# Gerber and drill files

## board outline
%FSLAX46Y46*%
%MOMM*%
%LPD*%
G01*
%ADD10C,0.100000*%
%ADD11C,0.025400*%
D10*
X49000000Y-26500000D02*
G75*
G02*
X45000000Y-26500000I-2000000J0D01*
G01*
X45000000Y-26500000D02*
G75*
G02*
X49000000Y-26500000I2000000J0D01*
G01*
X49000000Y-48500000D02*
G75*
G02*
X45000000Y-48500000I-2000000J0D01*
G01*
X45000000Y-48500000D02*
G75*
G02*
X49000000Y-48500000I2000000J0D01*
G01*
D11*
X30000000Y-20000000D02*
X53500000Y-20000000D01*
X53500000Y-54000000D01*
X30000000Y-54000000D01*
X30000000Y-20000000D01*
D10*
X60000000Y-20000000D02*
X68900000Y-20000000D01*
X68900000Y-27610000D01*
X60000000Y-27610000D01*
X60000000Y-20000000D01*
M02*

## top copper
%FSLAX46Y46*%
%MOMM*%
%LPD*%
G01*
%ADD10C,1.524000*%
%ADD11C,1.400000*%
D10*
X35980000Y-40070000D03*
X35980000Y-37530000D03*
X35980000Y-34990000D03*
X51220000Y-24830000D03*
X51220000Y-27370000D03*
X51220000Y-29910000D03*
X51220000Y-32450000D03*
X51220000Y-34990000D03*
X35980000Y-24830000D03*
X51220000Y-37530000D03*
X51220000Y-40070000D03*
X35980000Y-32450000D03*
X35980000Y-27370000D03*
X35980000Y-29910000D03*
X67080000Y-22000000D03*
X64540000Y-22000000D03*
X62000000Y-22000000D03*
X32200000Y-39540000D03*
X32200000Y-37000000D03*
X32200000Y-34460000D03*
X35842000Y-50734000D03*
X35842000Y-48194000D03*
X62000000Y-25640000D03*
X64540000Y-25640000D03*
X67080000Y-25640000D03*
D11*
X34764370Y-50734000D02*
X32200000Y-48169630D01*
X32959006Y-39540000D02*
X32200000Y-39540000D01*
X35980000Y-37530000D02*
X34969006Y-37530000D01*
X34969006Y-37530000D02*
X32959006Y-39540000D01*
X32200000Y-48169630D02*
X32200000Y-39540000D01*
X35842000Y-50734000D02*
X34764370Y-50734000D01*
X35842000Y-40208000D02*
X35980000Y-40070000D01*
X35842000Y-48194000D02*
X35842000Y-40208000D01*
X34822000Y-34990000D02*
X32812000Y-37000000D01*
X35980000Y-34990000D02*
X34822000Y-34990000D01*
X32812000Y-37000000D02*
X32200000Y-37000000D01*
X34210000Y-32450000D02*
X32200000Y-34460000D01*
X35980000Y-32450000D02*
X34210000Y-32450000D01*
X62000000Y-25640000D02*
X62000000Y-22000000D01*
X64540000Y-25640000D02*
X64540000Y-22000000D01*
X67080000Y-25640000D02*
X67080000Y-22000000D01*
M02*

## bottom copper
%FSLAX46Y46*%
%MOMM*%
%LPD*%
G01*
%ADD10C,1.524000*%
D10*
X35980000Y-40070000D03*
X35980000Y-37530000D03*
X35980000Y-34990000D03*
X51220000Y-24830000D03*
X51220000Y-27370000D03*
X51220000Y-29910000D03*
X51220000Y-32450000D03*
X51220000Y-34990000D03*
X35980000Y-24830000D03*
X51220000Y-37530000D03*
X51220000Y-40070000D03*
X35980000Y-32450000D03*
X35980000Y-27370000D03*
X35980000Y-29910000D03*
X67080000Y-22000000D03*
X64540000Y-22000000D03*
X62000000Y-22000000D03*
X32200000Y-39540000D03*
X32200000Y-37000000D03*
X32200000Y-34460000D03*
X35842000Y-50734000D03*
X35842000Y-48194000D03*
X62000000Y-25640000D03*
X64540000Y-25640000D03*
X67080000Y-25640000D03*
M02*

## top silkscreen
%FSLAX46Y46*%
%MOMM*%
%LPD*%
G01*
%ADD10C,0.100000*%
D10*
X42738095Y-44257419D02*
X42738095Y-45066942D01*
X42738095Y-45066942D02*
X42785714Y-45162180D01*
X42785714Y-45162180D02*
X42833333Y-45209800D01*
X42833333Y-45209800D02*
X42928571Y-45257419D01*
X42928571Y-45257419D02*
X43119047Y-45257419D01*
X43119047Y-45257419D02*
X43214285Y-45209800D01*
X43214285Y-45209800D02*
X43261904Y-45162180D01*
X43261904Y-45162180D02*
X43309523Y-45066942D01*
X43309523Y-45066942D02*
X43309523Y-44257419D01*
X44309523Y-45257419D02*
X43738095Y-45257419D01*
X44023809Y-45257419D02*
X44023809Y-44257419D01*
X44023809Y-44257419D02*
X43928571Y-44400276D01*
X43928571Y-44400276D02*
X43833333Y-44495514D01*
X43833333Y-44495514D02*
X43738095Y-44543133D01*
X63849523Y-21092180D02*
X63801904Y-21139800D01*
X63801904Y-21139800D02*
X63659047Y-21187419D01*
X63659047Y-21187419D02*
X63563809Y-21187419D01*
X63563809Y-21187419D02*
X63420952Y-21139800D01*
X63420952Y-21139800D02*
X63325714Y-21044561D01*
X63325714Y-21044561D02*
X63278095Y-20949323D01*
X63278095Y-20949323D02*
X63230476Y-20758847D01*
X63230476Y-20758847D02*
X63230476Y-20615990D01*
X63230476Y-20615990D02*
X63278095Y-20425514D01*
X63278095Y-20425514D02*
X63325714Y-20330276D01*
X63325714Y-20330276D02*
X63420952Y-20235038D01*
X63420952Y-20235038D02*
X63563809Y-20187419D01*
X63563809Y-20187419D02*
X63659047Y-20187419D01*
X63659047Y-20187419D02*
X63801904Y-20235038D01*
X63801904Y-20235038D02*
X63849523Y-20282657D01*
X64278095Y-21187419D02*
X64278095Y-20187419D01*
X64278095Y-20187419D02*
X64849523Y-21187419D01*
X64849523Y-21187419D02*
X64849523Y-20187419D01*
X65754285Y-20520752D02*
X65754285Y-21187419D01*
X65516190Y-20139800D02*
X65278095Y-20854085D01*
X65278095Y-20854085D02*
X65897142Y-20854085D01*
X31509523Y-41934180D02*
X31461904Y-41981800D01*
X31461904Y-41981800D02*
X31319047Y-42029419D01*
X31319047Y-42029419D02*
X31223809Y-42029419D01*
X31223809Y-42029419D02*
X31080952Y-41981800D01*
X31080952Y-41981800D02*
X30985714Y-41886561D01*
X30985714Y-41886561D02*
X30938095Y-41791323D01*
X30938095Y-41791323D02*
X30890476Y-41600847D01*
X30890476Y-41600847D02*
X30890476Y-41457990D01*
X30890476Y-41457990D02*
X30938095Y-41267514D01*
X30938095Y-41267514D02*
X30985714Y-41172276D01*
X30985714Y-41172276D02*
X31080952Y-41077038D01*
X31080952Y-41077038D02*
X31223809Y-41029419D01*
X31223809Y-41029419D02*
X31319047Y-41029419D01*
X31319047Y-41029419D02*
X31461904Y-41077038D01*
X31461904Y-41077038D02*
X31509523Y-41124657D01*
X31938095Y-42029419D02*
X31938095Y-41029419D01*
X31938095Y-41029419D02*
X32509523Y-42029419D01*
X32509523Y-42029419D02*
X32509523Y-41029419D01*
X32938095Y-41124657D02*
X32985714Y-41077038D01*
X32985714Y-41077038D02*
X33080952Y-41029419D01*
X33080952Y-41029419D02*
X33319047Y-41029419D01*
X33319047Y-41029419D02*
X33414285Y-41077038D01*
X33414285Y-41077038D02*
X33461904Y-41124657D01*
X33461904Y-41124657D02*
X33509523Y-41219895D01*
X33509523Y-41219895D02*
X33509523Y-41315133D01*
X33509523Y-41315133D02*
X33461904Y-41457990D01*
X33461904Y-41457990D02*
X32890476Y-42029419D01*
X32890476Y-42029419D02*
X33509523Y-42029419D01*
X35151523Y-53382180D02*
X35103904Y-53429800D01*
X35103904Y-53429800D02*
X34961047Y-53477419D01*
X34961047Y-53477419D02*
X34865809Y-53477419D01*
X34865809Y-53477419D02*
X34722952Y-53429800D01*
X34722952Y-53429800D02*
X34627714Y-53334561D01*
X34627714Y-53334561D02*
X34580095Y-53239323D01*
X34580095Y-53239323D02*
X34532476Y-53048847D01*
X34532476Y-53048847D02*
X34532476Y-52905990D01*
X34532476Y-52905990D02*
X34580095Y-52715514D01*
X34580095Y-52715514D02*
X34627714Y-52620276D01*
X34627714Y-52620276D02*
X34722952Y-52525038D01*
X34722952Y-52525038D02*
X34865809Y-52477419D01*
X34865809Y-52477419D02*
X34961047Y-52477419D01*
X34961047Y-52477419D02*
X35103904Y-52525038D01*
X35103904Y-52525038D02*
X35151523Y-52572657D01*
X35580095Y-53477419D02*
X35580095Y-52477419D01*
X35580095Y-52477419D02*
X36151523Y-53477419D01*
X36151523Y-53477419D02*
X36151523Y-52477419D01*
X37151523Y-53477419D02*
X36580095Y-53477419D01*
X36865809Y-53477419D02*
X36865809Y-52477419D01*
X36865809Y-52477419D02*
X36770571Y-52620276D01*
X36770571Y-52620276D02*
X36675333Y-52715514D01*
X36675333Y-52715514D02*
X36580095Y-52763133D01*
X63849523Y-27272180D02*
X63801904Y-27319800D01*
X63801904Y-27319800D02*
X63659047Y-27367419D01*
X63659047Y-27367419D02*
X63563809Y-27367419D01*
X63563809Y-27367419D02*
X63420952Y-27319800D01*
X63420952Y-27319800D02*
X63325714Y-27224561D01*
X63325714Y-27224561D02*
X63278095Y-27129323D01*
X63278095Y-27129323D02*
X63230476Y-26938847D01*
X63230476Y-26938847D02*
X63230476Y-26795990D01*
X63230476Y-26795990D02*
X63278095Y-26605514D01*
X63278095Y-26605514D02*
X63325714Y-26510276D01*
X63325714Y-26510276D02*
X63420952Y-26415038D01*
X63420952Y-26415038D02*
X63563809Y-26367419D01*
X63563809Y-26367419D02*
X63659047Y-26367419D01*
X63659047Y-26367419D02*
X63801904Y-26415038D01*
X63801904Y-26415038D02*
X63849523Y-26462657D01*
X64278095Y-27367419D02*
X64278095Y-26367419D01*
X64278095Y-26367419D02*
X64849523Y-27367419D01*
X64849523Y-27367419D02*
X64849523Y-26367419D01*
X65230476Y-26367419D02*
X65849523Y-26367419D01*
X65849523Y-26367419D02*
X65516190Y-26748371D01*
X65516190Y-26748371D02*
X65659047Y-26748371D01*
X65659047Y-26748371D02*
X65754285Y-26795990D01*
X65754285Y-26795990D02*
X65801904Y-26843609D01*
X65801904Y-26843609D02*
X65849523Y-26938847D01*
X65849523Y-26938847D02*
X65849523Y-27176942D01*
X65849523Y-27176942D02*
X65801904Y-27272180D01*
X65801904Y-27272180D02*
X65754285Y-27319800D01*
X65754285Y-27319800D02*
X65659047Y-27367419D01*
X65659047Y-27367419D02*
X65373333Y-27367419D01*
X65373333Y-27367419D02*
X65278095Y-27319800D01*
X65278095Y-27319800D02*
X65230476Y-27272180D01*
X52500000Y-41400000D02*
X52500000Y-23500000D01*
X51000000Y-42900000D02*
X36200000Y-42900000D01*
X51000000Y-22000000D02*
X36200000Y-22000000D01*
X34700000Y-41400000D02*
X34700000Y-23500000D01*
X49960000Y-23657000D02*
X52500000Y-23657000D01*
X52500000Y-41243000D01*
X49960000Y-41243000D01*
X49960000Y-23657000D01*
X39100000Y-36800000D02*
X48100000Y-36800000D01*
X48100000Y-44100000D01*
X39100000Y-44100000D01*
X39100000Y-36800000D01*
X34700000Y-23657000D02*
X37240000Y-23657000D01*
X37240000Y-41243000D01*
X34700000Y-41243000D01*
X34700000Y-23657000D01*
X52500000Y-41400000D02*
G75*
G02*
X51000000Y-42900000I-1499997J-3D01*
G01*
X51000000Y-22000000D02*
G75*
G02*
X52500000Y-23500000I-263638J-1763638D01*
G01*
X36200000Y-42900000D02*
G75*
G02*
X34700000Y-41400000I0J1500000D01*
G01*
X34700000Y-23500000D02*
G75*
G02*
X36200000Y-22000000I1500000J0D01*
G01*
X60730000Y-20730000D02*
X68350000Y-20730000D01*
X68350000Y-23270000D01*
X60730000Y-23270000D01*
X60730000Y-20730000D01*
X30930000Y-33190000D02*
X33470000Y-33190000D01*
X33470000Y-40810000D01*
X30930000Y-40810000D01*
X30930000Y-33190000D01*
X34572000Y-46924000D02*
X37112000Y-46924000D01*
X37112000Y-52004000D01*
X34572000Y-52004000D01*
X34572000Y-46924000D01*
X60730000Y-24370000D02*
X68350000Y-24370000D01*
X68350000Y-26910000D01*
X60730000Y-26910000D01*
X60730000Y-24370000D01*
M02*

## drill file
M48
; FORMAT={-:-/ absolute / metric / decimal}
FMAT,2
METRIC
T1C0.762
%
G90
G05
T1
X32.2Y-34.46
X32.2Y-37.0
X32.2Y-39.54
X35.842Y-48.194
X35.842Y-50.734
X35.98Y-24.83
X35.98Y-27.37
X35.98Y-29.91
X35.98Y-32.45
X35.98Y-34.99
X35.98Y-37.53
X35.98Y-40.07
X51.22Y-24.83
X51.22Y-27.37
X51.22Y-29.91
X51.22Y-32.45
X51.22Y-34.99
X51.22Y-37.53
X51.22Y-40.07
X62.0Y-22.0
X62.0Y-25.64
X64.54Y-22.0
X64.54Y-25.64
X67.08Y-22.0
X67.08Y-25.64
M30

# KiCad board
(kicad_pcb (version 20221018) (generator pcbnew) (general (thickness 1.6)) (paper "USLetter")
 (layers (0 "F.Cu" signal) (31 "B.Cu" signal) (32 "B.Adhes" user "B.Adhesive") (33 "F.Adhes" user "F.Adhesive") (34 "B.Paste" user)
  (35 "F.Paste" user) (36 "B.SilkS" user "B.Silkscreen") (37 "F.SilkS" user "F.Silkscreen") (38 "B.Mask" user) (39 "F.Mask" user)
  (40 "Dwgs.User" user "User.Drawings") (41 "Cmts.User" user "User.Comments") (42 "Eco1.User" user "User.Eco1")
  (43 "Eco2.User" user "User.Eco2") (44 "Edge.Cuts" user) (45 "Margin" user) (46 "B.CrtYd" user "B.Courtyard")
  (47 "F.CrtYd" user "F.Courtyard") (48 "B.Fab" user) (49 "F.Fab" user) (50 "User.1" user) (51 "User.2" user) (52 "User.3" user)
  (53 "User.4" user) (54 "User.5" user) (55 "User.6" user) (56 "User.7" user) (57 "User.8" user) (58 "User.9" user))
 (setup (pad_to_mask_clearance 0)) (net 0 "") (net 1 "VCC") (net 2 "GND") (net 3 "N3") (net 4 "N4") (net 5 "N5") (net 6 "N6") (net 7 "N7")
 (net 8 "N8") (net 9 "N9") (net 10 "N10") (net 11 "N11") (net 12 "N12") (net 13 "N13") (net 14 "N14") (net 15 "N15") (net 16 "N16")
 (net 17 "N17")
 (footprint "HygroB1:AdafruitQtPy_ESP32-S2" (layer "F.Cu") (at 43.6 32.45 180)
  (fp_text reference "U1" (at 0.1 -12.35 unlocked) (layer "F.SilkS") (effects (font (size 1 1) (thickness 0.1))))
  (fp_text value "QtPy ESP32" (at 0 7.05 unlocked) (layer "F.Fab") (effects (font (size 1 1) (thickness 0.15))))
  (fp_line (start -8.9 -8.95) (end -8.9 8.95) (stroke (width 0.1) (type default)) (layer "F.SilkS"))
  (fp_line (start -7.4 -10.45) (end 7.4 -10.45) (stroke (width 0.1) (type default)) (layer "F.SilkS"))
  (fp_line (start -7.4 10.45) (end 7.4 10.45) (stroke (width 0.1) (type default)) (layer "F.SilkS"))
  (fp_line (start 8.9 -8.95) (end 8.9 8.95) (stroke (width 0.1) (type default)) (layer "F.SilkS"))
  (fp_rect (start -8.9 -8.793) (end -6.36 8.793) (stroke (width 0.1) (type default)) (fill none) (layer "F.SilkS"))
  (fp_rect (start -4.5 -11.65) (end 4.5 -4.35) (stroke (width 0.1) (type default)) (fill none) (layer "F.SilkS"))
  (fp_rect (start 6.36 -8.793) (end 8.9 8.793) (stroke (width 0.1) (type default)) (fill none) (layer "F.SilkS"))
  (fp_arc (start -8.9 -8.95) (mid -8.460661 -10.010661) (end -7.4 -10.45) (stroke (width 0.1) (type default)) (layer "F.SilkS"))
  (fp_arc (start -7.4 10.45) (mid -8.397299 9.947299) (end -8.9 8.95) (stroke (width 0.1) (type default)) (layer "F.SilkS"))
  (fp_arc (start 7.4 -10.45) (mid 8.46066 -10.01066) (end 8.9 -8.95) (stroke (width 0.1) (type default)) (layer "F.SilkS"))
  (fp_arc (start 8.9 8.95) (mid 8.46066 10.01066) (end 7.4 10.45) (stroke (width 0.1) (type default)) (layer "F.SilkS"))
  (pad "0" thru_hole circle (at 7.62 -7.62 180) (size 1.524 1.524) (drill 0.762) (layers "*.Cu" "*.Mask") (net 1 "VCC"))
  (pad "2" thru_hole circle (at 7.62 -5.08 180) (size 1.524 1.524) (drill 0.762) (layers "*.Cu" "*.Mask") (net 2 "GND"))
  (pad "3" thru_hole circle (at 7.62 -2.54 180) (size 1.524 1.524) (drill 0.762) (layers "*.Cu" "*.Mask") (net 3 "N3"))
  (pad "5" thru_hole circle (at -7.62 7.62 180) (size 1.524 1.524) (drill 0.762) (layers "*.Cu" "*.Mask") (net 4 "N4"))
  (pad "6" thru_hole circle (at -7.62 5.08 180) (size 1.524 1.524) (drill 0.762) (layers "*.Cu" "*.Mask") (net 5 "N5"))
  (pad "7" thru_hole circle (at -7.62 2.54 180) (size 1.524 1.524) (drill 0.762) (layers "*.Cu" "*.Mask") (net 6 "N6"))
  (pad "8" thru_hole circle (at -7.62 0 180) (size 1.524 1.524) (drill 0.762) (layers "*.Cu" "*.Mask") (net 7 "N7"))
  (pad "9" thru_hole circle (at -7.62 -2.54 180) (size 1.524 1.524) (drill 0.762) (layers "*.Cu" "*.Mask") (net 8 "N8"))
  (pad "16" thru_hole circle (at 7.62 7.62 180) (size 1.524 1.524) (drill 0.762) (layers "*.Cu" "*.Mask") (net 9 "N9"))
  (pad "17" thru_hole circle (at -7.62 -5.08 180) (size 1.524 1.524) (drill 0.762) (layers "*.Cu" "*.Mask") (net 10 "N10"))
  (pad "18" thru_hole circle (at -7.62 -7.62 180) (size 1.524 1.524) (drill 0.762) (layers "*.Cu" "*.Mask") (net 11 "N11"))
  (pad "35" thru_hole circle (at 7.62 0 180) (size 1.524 1.524) (drill 0.762) (layers "*.Cu" "*.Mask") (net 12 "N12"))
  (pad "36" thru_hole circle (at 7.62 5.08 180) (size 1.524 1.524) (drill 0.762) (layers "*.Cu" "*.Mask") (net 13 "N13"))
  (pad "37" thru_hole circle (at 7.62 2.54 180) (size 1.524 1.524) (drill 0.762) (layers "*.Cu" "*.Mask") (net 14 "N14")))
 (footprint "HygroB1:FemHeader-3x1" (layer "F.Cu") (at 64.54 22 -90)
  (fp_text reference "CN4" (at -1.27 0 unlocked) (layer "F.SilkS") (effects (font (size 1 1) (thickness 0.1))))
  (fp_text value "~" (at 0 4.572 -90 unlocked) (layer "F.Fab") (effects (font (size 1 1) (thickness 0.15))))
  (fp_rect (start -1.27 -3.81) (end 1.27 3.81) (stroke (width 0.1) (type default)) (fill none) (layer "F.SilkS"))
  (pad "1" thru_hole circle (at 0 -2.54 270) (size 1.524 1.524) (drill 0.762) (layers "*.Cu" "*.Mask") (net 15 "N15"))
  (pad "2" thru_hole circle (at 0 0 270) (size 1.524 1.524) (drill 0.762) (layers "*.Cu" "*.Mask") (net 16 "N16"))
  (pad "3" thru_hole circle (at 0 2.54 270) (size 1.524 1.524) (drill 0.762) (layers "*.Cu" "*.Mask") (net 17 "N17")))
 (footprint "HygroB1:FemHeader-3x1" (layer "F.Cu") (at 32.2 37 180)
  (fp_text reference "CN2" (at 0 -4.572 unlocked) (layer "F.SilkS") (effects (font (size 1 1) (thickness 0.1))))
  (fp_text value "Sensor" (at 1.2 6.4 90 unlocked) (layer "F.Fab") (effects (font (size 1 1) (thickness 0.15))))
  (fp_rect (start -1.27 -3.81) (end 1.27 3.81) (stroke (width 0.1) (type default)) (fill none) (layer "F.SilkS"))
  (pad "1" thru_hole circle (at 0 -2.54 180) (size 1.524 1.524) (drill 0.762) (layers "*.Cu" "*.Mask") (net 2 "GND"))
  (pad "2" thru_hole circle (at 0 0 180) (size 1.524 1.524) (drill 0.762) (layers "*.Cu" "*.Mask") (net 3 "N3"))
  (pad "3" thru_hole circle (at 0 2.54 180) (size 1.524 1.524) (drill 0.762) (layers "*.Cu" "*.Mask") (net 12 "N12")))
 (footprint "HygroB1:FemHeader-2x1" (layer "F.Cu") (at 35.842 49.464 180)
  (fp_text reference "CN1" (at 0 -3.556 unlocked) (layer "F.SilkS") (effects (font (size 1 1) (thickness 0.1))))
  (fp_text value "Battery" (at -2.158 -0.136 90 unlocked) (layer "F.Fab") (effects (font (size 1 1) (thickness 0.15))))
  (fp_rect (start -1.27 -2.54) (end 1.27 2.54) (stroke (width 0.1) (type default)) (fill none) (layer "F.SilkS"))
  (pad "1" thru_hole circle (at 0 -1.27 180) (size 1.524 1.524) (drill 0.762) (layers "*.Cu" "*.Mask") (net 2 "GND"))
  (pad "2" thru_hole circle (at 0 1.27 180) (size 1.524 1.524) (drill 0.762) (layers "*.Cu" "*.Mask") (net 1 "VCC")))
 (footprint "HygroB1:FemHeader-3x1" (layer "F.Cu") (at 64.54 25.64 90)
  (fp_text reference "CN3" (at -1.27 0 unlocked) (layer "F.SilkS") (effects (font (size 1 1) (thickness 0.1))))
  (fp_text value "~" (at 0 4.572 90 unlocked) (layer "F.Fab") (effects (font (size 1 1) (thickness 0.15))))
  (fp_rect (start -1.27 -3.81) (end 1.27 3.81) (stroke (width 0.1) (type default)) (fill none) (layer "F.SilkS"))
  (pad "1" thru_hole circle (at 0 -2.54 90) (size 1.524 1.524) (drill 0.762) (layers "*.Cu" "*.Mask") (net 17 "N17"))
  (pad "2" thru_hole circle (at 0 0 90) (size 1.524 1.524) (drill 0.762) (layers "*.Cu" "*.Mask") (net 16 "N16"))
  (pad "3" thru_hole circle (at 0 2.54 90) (size 1.524 1.524) (drill 0.762) (layers "*.Cu" "*.Mask") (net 15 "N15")))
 (gr_circle (center 47 26.5) (end 49 26.5) (stroke (width 0.1) (type default)) (fill none) (layer "Edge.Cuts"))
 (gr_circle (center 47 48.5) (end 49 48.5) (stroke (width 0.1) (type default)) (fill none) (layer "Edge.Cuts"))
 (gr_rect (start 30 20) (end 53.5 54) (stroke (width 0.0254) (type default)) (fill none) (layer "Edge.Cuts"))
 (gr_rect (start 60 20) (end 68.9 27.61) (stroke (width 0.1) (type default)) (fill none) (layer "Edge.Cuts"))
 (segment (start 34.76437 50.734) (end 32.2 48.16963) (width 1.4) (layer "F.Cu") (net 2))
 (segment (start 32.959006 39.54) (end 32.2 39.54) (width 1.4) (layer "F.Cu") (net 2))
 (segment (start 35.98 37.53) (end 34.969006 37.53) (width 1.4) (layer "F.Cu") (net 2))
 (segment (start 34.969006 37.53) (end 32.959006 39.54) (width 1.4) (layer "F.Cu") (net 2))
 (segment (start 32.2 48.16963) (end 32.2 39.54) (width 1.4) (layer "F.Cu") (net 2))
 (segment (start 35.842 50.734) (end 34.76437 50.734) (width 1.4) (layer "F.Cu") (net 2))
 (segment (start 35.842 40.208) (end 35.98 40.07) (width 1.4) (layer "F.Cu") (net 1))
 (segment (start 35.842 48.194) (end 35.842 40.208) (width 1.4) (layer "F.Cu") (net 1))
 (segment (start 34.822 34.99) (end 32.812 37) (width 1.4) (layer "F.Cu") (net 3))
 (segment (start 35.98 34.99) (end 34.822 34.99) (width 1.4) (layer "F.Cu") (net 3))
 (segment (start 32.812 37) (end 32.2 37) (width 1.4) (layer "F.Cu") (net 3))
 (segment (start 34.21 32.45) (end 32.2 34.46) (width 1.4) (layer "F.Cu") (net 12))
 (segment (start 35.98 32.45) (end 34.21 32.45) (width 1.4) (layer "F.Cu") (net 12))
 (segment (start 62 25.64) (end 62 22) (width 1.4) (layer "F.Cu") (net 17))
 (segment (start 64.54 25.64) (end 64.54 22) (width 1.4) (layer "F.Cu") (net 16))
 (segment (start 67.08 25.64) (end 67.08 22) (width 1.4) (layer "F.Cu") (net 15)))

